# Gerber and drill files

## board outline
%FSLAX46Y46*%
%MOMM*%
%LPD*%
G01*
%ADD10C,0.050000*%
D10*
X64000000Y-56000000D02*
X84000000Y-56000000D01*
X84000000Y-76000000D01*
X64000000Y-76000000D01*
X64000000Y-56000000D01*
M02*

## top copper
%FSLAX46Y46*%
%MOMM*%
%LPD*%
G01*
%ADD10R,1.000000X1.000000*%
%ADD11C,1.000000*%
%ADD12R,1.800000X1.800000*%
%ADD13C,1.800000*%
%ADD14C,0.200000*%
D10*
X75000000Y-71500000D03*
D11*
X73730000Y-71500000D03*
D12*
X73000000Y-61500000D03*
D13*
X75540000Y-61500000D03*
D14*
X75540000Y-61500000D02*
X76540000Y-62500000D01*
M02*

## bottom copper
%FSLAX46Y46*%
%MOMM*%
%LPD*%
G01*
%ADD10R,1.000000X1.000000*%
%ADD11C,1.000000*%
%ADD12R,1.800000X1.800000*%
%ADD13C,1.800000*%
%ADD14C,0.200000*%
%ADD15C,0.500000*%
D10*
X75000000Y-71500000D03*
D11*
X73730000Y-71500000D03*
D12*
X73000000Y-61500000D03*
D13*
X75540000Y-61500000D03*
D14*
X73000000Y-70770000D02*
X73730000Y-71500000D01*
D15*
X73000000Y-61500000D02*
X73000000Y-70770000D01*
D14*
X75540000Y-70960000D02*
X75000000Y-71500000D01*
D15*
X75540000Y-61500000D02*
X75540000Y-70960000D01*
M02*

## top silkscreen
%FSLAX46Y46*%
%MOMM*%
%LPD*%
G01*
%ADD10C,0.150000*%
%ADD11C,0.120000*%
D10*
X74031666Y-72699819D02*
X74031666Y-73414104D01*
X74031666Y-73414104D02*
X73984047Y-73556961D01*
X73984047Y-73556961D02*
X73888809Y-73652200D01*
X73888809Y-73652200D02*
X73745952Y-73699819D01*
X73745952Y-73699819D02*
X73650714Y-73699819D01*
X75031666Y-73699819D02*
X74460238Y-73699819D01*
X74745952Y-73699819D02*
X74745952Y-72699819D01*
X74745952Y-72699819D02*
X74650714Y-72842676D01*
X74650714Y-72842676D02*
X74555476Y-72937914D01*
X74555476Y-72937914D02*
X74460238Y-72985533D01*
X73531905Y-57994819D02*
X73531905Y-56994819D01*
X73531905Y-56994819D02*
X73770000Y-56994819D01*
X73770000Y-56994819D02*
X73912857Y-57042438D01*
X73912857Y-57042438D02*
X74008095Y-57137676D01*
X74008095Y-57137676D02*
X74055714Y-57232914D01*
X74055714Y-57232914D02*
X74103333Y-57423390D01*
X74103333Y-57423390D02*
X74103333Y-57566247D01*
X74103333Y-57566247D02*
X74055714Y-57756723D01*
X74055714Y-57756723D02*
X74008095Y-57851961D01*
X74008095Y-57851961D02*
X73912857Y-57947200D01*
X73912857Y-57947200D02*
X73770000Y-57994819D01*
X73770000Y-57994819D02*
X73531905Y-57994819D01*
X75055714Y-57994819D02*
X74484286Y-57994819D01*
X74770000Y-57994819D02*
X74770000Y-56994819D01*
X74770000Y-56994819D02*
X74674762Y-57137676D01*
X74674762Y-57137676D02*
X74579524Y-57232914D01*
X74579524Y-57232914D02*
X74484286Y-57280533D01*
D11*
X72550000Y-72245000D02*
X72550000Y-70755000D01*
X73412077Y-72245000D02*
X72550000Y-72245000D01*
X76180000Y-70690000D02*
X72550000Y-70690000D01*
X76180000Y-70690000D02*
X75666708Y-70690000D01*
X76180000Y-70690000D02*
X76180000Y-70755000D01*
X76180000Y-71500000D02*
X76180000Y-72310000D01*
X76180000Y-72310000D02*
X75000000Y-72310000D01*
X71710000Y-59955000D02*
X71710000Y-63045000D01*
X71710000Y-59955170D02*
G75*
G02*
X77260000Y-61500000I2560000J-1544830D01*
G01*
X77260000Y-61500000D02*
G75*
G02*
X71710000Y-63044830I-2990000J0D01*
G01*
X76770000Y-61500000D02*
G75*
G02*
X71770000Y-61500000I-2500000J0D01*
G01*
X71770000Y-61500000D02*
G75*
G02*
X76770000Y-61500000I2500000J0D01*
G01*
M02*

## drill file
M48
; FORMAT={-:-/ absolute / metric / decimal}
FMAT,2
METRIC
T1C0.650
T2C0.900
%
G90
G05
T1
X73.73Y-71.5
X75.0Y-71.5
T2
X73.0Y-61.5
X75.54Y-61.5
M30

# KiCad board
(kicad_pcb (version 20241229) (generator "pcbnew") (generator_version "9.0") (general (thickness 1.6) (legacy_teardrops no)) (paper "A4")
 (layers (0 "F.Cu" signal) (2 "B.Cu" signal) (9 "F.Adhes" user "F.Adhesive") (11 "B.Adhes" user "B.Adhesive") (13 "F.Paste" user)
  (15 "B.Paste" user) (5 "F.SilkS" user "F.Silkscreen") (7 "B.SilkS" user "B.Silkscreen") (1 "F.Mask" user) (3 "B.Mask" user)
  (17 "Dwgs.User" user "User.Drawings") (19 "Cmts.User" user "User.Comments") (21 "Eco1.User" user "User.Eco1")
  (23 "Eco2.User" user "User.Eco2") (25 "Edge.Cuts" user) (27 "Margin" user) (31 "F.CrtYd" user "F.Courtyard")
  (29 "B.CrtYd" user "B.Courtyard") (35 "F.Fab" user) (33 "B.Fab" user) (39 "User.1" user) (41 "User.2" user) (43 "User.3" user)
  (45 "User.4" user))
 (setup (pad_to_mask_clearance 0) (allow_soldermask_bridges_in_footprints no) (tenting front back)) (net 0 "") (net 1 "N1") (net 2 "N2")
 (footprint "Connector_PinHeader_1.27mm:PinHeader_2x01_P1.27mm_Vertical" (layer "F.Cu") (at 75 71.5 180)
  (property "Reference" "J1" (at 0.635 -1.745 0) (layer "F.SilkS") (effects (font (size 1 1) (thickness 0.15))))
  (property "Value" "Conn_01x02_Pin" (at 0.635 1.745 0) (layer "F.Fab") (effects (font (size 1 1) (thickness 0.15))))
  (fp_line (start 2.45 -0.745) (end 2.45 0.745) (stroke (width 0.12) (type solid)) (layer "F.SilkS"))
  (fp_line (start 1.587923 -0.745) (end 2.45 -0.745) (stroke (width 0.12) (type solid)) (layer "F.SilkS"))
  (fp_line (start -1.18 0.81) (end 2.45 0.81) (stroke (width 0.12) (type solid)) (layer "F.SilkS"))
  (fp_line (start -1.18 0.81) (end -0.666708 0.81) (stroke (width 0.12) (type solid)) (layer "F.SilkS"))
  (fp_line (start -1.18 0.81) (end -1.18 0.745) (stroke (width 0.12) (type solid)) (layer "F.SilkS"))
  (fp_line (start -1.18 0) (end -1.18 -0.81) (stroke (width 0.12) (type solid)) (layer "F.SilkS"))
  (fp_line (start -1.18 -0.81) (end 0 -0.81) (stroke (width 0.12) (type solid)) (layer "F.SilkS"))
  (pad "1" thru_hole rect (at 0 0 180) (size 1 1) (drill 0.65) (layers "*.Cu" "*.Mask") (remove_unused_layers no) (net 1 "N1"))
  (pad "2" thru_hole circle (at 1.27 0 180) (size 1 1) (drill 0.65) (layers "*.Cu" "*.Mask") (remove_unused_layers no) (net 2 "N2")))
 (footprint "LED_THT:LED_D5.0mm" (layer "F.Cu") (at 73 61.5)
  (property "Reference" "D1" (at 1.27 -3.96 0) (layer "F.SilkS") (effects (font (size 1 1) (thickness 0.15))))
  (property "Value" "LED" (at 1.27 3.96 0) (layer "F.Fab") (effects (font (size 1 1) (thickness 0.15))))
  (fp_line (start -1.29 -1.545) (end -1.29 1.545) (stroke (width 0.12) (type solid)) (layer "F.SilkS"))
  (fp_arc (start -1.29 -1.54483) (mid 2.071779 -2.880495) (end 4.26 0) (stroke (width 0.12) (type solid)) (layer "F.SilkS"))
  (fp_arc (start 4.26 0) (mid 2.071779 2.880495) (end -1.29 1.54483) (stroke (width 0.12) (type solid)) (layer "F.SilkS"))
  (fp_circle (center 1.27 0) (end 3.77 0) (stroke (width 0.12) (type solid)) (fill no) (layer "F.SilkS"))
  (pad "1" thru_hole rect (at 0 0) (size 1.8 1.8) (drill 0.9) (layers "*.Cu" "*.Mask") (remove_unused_layers no) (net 2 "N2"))
  (pad "2" thru_hole circle (at 2.54 0) (size 1.8 1.8) (drill 0.9) (layers "*.Cu" "*.Mask") (remove_unused_layers no) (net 1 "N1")))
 (gr_rect (start 64 56) (end 84 76) (stroke (width 0.05) (type solid)) (fill no) (layer "Edge.Cuts"))
 (segment (start 73 70.77) (end 73.73 71.5) (width 0.2) (layer "B.Cu") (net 2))
 (segment (start 73 61.5) (end 73 70.77) (width 0.5) (layer "B.Cu") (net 2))
 (segment (start 75.54 61.5) (end 76.54 62.5) (width 0.2) (layer "F.Cu") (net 1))
 (segment (start 75.54 70.96) (end 75 71.5) (width 0.2) (layer "B.Cu") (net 1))
 (segment (start 75.54 61.5) (end 75.54 70.96) (width 0.5) (layer "B.Cu") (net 1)))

